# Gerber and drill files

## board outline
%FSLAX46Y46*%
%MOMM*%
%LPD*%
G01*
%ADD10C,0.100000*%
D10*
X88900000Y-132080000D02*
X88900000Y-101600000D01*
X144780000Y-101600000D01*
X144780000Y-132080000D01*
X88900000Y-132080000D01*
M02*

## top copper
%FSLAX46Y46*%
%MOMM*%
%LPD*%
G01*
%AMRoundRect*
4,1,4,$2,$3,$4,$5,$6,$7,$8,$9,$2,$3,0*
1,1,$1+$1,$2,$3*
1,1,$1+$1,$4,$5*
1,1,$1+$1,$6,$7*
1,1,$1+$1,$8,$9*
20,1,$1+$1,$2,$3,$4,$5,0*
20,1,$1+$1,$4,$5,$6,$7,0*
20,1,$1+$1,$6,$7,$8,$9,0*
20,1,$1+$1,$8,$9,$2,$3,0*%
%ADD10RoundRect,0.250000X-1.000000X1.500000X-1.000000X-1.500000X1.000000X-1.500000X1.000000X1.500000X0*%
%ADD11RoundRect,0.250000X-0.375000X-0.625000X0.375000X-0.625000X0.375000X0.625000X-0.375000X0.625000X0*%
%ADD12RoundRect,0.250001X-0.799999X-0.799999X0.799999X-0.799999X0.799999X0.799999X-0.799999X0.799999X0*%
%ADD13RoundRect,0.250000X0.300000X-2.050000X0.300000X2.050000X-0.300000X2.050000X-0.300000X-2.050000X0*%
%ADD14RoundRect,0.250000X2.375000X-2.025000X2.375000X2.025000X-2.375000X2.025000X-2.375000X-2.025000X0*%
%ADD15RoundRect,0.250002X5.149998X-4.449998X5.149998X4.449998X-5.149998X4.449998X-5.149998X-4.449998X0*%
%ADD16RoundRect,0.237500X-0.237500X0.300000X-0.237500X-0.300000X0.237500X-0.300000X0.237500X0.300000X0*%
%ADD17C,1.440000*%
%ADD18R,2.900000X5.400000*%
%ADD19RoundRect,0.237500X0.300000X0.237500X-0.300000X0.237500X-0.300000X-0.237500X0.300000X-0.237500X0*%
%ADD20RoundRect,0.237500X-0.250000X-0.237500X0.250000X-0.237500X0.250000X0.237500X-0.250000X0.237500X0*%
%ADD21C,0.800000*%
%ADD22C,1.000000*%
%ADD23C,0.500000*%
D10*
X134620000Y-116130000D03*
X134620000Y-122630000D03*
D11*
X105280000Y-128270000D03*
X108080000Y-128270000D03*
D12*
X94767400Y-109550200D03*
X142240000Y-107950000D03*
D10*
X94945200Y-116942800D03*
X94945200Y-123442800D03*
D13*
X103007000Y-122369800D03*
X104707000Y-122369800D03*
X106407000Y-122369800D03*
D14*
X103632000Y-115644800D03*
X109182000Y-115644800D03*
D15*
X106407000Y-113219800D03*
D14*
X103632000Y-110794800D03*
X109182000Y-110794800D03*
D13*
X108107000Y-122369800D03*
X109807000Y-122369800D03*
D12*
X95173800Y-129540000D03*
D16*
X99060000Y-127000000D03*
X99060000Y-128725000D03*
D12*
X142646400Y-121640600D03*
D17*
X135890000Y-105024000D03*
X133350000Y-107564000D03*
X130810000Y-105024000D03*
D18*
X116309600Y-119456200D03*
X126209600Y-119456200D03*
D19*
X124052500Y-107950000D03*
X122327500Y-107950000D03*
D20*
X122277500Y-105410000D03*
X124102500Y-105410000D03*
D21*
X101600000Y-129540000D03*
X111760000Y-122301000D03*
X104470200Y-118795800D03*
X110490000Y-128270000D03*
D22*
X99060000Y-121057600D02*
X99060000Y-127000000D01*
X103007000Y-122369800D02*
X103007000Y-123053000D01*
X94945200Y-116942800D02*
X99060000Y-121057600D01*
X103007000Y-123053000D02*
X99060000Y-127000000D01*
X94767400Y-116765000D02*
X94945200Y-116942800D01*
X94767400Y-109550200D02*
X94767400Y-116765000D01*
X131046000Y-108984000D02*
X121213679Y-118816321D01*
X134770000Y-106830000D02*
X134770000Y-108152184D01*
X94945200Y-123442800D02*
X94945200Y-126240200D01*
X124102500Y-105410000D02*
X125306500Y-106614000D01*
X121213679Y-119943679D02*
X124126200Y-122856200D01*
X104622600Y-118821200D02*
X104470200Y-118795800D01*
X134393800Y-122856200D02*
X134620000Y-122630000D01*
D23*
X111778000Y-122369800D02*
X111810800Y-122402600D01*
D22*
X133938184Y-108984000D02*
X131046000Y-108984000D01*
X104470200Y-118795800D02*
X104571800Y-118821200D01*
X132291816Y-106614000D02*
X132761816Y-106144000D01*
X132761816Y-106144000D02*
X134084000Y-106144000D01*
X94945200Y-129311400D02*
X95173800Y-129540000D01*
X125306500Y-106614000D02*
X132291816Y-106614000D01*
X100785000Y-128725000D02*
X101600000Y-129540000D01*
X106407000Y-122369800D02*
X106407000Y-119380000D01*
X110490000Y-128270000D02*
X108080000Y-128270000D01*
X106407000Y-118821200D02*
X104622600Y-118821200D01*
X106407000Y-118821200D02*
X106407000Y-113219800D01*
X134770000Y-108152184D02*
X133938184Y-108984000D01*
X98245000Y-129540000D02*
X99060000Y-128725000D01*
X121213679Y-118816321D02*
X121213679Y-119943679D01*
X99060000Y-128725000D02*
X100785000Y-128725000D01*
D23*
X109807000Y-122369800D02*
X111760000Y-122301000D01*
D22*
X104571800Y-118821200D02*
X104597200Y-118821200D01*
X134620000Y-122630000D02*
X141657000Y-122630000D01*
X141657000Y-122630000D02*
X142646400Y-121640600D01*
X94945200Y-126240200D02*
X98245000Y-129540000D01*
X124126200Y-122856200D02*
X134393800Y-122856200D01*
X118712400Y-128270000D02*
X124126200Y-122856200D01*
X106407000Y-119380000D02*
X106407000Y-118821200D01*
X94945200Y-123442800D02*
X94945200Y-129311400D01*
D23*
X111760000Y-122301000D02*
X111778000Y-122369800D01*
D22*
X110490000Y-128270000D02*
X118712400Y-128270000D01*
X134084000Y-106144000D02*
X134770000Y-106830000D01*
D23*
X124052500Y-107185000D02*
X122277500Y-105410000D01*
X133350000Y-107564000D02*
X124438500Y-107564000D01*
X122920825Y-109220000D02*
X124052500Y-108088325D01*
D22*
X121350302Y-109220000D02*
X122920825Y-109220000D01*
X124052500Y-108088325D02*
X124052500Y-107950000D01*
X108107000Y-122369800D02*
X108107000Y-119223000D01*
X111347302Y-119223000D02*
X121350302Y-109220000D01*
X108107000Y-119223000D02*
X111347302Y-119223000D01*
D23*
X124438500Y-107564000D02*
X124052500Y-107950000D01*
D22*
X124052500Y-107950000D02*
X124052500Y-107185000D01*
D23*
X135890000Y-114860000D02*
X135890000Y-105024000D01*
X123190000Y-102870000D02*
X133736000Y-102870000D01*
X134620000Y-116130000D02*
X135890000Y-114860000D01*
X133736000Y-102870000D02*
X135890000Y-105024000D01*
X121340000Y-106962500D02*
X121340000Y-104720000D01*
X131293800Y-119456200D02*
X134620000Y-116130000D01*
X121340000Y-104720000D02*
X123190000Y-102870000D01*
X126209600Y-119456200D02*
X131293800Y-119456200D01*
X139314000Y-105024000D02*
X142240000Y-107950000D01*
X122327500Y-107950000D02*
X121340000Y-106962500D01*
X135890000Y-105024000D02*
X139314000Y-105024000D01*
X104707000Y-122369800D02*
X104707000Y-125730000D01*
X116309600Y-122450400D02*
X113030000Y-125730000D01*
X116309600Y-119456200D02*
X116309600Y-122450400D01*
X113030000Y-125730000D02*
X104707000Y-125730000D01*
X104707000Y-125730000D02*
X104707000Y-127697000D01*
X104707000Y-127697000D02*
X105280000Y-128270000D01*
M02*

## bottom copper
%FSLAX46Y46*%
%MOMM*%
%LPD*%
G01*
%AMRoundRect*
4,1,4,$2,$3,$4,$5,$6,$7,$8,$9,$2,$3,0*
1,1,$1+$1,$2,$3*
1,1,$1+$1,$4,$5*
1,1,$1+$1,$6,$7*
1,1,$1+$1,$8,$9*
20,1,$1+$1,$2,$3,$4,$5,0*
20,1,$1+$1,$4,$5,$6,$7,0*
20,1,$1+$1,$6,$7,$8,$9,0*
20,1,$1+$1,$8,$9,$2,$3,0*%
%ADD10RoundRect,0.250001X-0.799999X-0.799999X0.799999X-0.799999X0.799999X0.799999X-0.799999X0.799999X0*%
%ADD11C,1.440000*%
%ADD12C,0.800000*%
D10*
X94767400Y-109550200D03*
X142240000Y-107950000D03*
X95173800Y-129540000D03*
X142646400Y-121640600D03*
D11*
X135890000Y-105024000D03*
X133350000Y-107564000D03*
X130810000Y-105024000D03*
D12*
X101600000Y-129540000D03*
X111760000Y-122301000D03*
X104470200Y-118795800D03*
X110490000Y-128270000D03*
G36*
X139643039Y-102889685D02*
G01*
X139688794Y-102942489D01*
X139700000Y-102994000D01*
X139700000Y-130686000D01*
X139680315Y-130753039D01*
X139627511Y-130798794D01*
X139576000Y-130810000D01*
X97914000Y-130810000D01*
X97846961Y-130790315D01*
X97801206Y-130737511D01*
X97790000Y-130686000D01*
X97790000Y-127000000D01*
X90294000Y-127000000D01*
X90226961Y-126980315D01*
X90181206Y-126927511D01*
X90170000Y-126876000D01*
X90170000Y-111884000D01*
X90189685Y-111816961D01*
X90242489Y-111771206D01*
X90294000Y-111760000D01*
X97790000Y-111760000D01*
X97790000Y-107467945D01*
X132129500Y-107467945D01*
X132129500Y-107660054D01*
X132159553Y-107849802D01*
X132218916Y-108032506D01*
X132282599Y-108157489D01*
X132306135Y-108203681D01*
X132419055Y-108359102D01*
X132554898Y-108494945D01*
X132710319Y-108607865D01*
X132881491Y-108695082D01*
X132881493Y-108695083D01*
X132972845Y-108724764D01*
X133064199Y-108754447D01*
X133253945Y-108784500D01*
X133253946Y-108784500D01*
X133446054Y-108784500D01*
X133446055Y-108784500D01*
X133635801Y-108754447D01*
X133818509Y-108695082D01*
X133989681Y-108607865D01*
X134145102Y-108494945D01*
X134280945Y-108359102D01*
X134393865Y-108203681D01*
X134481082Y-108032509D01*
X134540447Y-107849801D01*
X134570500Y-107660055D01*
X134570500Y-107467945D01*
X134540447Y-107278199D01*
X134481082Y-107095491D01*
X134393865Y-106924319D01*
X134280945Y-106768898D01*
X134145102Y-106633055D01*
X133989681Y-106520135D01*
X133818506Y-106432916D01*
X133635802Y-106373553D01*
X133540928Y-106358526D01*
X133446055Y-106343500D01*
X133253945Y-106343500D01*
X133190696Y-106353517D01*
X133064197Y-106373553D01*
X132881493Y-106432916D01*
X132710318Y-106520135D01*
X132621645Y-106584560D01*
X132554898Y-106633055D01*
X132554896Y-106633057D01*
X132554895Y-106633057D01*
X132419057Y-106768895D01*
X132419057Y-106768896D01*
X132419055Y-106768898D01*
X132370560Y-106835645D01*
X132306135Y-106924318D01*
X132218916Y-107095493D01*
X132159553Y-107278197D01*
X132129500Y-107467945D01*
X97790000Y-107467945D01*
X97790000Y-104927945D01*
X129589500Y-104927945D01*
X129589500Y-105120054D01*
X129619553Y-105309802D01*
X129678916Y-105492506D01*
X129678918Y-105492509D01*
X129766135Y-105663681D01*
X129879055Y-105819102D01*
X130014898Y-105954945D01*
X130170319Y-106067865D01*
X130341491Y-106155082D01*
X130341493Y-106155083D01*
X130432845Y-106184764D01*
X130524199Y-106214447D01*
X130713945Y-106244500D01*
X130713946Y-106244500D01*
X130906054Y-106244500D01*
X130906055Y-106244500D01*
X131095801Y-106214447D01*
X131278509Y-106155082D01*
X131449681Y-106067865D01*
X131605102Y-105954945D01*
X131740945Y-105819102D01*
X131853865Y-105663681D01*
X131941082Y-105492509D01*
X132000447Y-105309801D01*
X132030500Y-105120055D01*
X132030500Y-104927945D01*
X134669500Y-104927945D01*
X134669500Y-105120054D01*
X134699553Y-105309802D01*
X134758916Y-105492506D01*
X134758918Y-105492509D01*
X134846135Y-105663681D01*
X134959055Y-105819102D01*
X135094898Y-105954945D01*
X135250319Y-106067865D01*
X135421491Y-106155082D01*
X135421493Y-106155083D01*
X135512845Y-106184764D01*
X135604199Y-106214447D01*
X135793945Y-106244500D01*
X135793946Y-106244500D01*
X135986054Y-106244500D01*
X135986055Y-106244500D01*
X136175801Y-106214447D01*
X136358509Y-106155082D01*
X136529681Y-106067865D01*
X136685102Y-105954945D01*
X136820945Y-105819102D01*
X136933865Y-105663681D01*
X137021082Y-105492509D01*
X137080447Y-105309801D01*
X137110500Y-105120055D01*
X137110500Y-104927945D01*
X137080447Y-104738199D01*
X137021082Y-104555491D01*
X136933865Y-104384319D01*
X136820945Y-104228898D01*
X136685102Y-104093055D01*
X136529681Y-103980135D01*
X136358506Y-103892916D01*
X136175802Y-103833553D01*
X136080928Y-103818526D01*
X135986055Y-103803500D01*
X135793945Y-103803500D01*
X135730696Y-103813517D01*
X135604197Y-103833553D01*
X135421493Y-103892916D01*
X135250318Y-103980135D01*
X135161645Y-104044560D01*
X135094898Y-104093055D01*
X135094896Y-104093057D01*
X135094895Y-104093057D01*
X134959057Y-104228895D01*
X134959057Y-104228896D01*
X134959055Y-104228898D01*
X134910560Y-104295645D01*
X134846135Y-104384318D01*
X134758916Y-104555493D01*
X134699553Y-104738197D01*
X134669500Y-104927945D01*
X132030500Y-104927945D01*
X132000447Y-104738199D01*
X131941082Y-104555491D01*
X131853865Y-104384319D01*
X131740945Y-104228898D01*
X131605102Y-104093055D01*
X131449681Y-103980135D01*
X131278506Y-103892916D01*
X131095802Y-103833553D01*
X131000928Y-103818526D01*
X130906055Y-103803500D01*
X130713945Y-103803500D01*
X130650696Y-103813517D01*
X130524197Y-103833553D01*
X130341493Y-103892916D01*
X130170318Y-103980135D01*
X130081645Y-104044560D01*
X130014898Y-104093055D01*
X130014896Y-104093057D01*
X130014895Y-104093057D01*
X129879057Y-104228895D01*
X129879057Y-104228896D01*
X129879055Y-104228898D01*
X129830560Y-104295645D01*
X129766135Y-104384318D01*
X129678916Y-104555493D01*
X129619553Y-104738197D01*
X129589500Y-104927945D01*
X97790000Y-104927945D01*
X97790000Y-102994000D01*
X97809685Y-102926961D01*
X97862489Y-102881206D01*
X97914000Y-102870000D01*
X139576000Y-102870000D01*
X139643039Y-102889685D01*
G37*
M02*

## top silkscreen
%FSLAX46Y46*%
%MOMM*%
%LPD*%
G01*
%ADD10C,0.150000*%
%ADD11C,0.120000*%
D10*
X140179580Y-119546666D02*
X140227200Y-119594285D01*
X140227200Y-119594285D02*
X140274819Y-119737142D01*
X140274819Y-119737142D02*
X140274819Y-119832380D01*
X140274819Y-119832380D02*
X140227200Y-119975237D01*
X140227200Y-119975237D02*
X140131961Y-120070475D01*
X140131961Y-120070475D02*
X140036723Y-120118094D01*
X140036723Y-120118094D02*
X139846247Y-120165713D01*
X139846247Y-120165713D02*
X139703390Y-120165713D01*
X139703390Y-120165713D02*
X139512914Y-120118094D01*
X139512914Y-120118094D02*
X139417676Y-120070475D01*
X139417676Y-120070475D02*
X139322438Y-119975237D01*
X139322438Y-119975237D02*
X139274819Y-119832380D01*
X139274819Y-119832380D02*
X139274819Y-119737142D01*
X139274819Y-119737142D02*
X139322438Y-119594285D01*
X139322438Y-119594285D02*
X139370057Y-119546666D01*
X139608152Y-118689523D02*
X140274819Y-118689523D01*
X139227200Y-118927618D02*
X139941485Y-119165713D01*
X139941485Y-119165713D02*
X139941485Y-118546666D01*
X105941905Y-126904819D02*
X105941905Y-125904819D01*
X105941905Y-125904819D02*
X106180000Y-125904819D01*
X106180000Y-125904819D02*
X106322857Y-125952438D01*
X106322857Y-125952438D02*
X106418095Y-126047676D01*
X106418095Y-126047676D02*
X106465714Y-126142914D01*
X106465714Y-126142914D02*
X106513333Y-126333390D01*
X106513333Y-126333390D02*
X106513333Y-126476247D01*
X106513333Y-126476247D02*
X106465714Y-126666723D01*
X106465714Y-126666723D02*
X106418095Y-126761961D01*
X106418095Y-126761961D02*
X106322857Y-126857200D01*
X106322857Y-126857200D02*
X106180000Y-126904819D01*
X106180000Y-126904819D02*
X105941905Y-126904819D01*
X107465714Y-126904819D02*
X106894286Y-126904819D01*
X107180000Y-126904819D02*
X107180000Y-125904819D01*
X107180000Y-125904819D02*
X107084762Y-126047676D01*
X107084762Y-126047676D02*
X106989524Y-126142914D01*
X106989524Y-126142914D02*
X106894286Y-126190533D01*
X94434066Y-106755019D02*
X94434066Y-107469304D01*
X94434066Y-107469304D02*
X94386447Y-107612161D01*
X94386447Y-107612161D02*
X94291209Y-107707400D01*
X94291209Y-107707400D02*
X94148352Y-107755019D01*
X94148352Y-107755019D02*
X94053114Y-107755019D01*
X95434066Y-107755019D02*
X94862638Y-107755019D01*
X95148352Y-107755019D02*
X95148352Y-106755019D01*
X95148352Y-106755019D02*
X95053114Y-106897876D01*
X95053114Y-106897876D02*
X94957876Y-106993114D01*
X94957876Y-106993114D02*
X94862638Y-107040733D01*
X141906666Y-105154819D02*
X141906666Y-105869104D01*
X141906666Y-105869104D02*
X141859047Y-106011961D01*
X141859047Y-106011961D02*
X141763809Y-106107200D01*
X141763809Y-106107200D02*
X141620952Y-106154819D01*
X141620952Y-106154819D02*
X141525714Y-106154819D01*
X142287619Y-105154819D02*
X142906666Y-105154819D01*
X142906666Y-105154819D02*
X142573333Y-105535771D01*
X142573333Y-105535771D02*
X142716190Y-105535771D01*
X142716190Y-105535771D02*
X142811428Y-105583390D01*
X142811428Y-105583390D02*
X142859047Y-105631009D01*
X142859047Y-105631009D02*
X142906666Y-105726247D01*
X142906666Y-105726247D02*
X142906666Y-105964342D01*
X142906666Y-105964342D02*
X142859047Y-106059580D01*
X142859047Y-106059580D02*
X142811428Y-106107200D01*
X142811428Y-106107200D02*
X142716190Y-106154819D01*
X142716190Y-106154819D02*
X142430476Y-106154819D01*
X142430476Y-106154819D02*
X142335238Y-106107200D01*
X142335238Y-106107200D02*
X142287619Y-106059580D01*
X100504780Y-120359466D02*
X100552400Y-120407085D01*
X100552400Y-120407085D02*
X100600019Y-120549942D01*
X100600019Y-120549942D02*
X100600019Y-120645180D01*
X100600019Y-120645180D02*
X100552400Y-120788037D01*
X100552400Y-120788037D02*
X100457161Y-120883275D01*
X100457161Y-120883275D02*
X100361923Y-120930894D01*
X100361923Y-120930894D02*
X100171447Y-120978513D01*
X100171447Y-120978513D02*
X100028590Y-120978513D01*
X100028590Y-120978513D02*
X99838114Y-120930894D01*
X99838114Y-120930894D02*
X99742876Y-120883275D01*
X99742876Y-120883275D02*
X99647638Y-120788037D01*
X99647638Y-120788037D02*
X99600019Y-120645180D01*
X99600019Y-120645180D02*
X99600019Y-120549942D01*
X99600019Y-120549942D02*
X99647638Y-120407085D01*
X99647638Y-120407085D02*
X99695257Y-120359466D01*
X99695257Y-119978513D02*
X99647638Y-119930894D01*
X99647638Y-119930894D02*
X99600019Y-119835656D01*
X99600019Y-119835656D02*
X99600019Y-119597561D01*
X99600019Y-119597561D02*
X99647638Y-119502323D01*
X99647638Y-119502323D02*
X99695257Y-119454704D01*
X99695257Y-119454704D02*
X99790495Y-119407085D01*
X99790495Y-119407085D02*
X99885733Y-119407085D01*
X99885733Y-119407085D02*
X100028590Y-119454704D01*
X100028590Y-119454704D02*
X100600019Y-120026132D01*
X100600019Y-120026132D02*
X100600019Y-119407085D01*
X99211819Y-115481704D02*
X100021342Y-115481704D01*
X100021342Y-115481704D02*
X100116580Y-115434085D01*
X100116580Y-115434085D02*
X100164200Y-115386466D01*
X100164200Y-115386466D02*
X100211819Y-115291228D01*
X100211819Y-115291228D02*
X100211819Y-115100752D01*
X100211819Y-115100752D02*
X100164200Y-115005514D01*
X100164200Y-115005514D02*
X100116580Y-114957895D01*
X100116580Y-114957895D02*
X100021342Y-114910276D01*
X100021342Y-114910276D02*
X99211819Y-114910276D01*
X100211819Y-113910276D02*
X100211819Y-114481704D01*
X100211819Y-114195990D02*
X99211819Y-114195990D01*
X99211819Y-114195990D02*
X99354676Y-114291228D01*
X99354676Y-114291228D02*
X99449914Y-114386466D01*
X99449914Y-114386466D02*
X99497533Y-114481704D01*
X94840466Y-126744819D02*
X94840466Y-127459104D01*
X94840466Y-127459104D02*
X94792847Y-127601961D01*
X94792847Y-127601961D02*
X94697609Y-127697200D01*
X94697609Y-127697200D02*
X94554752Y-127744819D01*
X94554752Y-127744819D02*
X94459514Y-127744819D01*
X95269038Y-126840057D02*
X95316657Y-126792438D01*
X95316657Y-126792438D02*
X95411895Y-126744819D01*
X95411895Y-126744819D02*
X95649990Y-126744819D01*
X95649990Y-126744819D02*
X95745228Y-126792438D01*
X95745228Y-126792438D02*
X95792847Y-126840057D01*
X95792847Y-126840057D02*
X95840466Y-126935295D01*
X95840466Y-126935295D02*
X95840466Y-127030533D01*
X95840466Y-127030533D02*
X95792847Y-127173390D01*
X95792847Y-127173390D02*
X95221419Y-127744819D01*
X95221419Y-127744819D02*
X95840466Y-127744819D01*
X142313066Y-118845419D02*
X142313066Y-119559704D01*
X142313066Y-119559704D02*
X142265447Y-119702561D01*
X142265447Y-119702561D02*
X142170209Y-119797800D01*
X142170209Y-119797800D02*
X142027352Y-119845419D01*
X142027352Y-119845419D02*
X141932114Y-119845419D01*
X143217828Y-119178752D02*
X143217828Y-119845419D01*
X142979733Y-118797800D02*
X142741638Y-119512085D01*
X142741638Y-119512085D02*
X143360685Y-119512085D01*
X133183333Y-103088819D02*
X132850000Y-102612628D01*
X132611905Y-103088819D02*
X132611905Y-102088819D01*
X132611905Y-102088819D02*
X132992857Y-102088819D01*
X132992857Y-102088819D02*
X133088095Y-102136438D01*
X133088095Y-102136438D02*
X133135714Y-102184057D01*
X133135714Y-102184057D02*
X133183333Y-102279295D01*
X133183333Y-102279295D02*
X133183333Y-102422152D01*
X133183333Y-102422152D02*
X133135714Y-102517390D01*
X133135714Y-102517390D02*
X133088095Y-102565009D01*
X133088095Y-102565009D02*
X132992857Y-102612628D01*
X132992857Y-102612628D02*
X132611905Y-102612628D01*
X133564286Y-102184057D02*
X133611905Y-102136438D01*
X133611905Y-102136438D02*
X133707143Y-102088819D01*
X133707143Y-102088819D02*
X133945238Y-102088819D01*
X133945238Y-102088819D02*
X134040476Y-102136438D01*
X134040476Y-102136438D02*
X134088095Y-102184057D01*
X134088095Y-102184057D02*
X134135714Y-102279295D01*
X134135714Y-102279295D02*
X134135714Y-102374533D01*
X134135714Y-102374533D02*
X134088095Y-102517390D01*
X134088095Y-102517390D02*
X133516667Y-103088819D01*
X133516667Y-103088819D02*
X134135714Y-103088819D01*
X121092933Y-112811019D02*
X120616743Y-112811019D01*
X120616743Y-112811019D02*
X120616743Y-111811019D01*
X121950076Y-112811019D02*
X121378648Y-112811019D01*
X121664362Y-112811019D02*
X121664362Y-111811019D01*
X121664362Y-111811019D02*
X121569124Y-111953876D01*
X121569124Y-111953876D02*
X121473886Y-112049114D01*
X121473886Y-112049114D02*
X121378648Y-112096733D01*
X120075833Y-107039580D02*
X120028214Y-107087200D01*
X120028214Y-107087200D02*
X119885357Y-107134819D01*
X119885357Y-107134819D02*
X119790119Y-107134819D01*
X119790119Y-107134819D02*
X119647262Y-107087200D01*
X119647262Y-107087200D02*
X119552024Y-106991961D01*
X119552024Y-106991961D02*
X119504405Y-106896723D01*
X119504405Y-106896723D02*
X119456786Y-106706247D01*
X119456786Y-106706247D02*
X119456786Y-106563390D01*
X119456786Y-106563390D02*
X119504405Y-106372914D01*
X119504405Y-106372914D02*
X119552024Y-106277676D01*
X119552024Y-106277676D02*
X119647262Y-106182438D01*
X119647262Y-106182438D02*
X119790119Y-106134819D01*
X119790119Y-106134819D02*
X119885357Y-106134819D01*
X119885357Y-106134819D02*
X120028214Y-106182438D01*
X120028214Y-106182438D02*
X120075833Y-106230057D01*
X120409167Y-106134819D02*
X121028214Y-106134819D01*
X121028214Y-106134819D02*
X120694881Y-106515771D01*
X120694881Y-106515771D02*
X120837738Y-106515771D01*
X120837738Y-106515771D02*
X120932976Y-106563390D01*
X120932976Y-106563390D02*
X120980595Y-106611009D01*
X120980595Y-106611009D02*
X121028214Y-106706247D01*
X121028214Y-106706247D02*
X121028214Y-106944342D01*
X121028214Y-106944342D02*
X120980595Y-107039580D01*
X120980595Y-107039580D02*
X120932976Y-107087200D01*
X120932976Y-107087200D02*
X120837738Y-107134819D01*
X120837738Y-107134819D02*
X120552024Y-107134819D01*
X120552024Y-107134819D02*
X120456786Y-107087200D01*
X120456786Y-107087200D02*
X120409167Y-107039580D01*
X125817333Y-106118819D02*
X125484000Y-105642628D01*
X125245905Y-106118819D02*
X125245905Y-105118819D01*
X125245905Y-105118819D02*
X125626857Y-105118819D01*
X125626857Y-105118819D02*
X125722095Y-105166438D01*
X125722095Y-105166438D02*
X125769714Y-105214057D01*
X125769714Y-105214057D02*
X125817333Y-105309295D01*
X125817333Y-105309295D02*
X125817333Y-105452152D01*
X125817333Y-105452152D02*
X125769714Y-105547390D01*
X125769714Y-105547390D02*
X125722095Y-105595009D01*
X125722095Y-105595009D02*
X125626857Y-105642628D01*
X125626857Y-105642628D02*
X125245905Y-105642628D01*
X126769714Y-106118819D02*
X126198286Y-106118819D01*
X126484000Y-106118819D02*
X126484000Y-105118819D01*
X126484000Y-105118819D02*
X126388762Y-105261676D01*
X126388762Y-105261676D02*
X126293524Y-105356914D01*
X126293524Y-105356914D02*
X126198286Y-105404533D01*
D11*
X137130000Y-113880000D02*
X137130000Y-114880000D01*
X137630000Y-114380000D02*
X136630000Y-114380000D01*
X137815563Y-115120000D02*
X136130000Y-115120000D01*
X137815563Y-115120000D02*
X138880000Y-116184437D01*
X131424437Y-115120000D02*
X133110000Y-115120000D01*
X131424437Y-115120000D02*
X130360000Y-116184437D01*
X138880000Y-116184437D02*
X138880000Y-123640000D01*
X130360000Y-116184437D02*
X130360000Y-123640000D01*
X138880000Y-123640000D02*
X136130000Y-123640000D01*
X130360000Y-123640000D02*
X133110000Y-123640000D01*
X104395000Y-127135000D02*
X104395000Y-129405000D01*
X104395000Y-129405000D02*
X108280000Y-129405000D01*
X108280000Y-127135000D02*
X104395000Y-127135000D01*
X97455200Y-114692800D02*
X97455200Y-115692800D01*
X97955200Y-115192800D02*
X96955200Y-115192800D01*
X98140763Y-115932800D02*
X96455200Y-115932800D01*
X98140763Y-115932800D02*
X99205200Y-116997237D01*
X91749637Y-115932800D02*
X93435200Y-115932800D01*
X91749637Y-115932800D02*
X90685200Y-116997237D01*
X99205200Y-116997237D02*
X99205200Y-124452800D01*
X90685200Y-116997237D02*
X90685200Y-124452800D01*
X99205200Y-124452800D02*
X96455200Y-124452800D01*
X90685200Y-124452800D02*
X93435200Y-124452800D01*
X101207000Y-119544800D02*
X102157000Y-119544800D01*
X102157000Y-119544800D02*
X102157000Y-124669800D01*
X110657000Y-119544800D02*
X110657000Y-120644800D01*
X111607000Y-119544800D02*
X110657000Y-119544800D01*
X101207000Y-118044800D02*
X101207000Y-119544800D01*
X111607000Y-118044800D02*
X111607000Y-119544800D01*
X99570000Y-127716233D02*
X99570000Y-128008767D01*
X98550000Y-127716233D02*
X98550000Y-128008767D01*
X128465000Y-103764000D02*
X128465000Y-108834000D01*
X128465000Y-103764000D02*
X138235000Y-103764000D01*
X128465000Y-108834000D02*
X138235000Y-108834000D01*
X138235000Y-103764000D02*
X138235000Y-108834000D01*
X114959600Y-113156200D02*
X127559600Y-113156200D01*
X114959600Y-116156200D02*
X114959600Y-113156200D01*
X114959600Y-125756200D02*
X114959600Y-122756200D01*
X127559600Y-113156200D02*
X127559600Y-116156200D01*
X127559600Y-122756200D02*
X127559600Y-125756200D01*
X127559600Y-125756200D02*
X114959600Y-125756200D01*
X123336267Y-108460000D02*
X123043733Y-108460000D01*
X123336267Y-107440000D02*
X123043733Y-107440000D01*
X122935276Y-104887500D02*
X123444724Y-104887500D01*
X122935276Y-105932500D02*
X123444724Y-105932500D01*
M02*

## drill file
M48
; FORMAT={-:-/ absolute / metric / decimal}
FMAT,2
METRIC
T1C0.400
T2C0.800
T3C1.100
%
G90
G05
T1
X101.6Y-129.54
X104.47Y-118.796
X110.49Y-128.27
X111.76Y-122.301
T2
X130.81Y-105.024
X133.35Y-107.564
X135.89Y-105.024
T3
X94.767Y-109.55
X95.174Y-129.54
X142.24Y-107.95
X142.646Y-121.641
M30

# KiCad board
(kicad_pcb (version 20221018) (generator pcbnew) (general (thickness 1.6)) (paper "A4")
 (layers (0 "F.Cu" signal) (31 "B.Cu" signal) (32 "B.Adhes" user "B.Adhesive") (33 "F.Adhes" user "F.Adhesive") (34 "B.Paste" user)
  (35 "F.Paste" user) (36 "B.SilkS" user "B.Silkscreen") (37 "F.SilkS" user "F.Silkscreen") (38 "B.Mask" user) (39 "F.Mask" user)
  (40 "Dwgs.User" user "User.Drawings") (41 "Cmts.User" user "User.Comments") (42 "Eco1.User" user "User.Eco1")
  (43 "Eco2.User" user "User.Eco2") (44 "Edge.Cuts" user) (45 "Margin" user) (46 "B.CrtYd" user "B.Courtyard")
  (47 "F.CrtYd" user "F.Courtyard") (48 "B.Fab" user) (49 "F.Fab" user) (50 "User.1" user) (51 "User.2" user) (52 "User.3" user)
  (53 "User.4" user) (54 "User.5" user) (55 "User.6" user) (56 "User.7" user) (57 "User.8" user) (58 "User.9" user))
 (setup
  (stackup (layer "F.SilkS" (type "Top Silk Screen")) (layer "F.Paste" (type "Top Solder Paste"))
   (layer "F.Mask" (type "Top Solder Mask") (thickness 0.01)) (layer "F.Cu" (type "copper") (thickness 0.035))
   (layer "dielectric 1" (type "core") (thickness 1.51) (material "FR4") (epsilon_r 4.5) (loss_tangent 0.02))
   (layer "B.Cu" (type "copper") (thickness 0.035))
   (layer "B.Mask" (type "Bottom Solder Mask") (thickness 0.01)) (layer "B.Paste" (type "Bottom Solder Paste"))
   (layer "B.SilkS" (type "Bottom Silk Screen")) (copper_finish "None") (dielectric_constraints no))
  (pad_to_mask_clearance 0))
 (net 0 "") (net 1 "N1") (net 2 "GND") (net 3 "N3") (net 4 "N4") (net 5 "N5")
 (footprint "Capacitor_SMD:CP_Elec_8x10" (layer "F.Cu") (at 134.62 119.38 -90)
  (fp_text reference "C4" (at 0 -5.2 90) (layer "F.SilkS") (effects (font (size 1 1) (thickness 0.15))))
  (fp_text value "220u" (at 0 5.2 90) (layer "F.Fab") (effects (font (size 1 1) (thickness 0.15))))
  (fp_line (start -5.5 -2.51) (end -4.5 -2.51) (stroke (width 0.12) (type solid)) (layer "F.SilkS"))
  (fp_line (start -5 -3.01) (end -5 -2.01) (stroke (width 0.12) (type solid)) (layer "F.SilkS"))
  (fp_line (start -4.26 -3.195563) (end -4.26 -1.51) (stroke (width 0.12) (type solid)) (layer "F.SilkS"))
  (fp_line (start -4.26 -3.195563) (end -3.195563 -4.26) (stroke (width 0.12) (type solid)) (layer "F.SilkS"))
  (fp_line (start -4.26 3.195563) (end -4.26 1.51) (stroke (width 0.12) (type solid)) (layer "F.SilkS"))
  (fp_line (start -4.26 3.195563) (end -3.195563 4.26) (stroke (width 0.12) (type solid)) (layer "F.SilkS"))
  (fp_line (start -3.195563 -4.26) (end 4.26 -4.26) (stroke (width 0.12) (type solid)) (layer "F.SilkS"))
  (fp_line (start -3.195563 4.26) (end 4.26 4.26) (stroke (width 0.12) (type solid)) (layer "F.SilkS"))
  (fp_line (start 4.26 -4.26) (end 4.26 -1.51) (stroke (width 0.12) (type solid)) (layer "F.SilkS"))
  (fp_line (start 4.26 4.26) (end 4.26 1.51) (stroke (width 0.12) (type solid)) (layer "F.SilkS"))
  (pad "1" smd roundrect (at -3.25 0 270) (size 3.5 2.5) (layers "F.Cu" "F.Paste" "F.Mask") (roundrect_rratio 0.1) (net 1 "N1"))
  (pad "2" smd roundrect (at 3.25 0 270) (size 3.5 2.5) (layers "F.Cu" "F.Paste" "F.Mask") (roundrect_rratio 0.1) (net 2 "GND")))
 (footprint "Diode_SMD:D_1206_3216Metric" (layer "F.Cu") (at 106.68 128.27)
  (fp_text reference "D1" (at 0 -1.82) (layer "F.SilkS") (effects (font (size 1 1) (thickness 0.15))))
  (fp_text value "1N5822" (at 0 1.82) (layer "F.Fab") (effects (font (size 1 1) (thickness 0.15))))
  (fp_line (start -2.285 -1.135) (end -2.285 1.135) (stroke (width 0.12) (type solid)) (layer "F.SilkS"))
  (fp_line (start -2.285 1.135) (end 1.6 1.135) (stroke (width 0.12) (type solid)) (layer "F.SilkS"))
  (fp_line (start 1.6 -1.135) (end -2.285 -1.135) (stroke (width 0.12) (type solid)) (layer "F.SilkS"))
  (pad "1" smd roundrect (at -1.4 0) (size 1.25 1.75) (layers "F.Cu" "F.Paste" "F.Mask") (roundrect_rratio 0.2) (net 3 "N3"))
  (pad "2" smd roundrect (at 1.4 0) (size 1.25 1.75) (layers "F.Cu" "F.Paste" "F.Mask") (roundrect_rratio 0.2) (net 2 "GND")))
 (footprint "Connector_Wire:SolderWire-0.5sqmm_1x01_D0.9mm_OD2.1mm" (layer "F.Cu") (at 94.7674 109.5502)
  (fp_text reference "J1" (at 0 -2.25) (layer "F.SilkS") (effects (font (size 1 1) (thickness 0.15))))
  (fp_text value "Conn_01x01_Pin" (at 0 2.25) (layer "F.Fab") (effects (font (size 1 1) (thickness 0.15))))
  (pad "1" thru_hole roundrect (at 0 0) (size 2.1 2.1) (drill 1.1) (layers "*.Cu" "*.Mask") (roundrect_rratio 0.119048) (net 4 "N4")))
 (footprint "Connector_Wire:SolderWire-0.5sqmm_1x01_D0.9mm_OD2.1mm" (layer "F.Cu") (at 142.24 107.95)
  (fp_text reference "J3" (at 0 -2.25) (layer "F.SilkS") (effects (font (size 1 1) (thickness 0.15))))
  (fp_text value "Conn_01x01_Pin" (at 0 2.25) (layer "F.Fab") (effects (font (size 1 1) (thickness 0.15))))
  (pad "1" thru_hole roundrect (at 0 0) (size 2.1 2.1) (drill 1.1) (layers "*.Cu" "*.Mask") (roundrect_rratio 0.119048) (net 1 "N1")))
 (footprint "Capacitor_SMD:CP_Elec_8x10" (layer "F.Cu") (at 94.9452 120.1928 -90)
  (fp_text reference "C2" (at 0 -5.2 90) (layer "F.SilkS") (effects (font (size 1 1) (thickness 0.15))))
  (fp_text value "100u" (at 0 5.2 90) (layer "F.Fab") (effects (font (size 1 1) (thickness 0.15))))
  (fp_line (start -5.5 -2.51) (end -4.5 -2.51) (stroke (width 0.12) (type solid)) (layer "F.SilkS"))
  (fp_line (start -5 -3.01) (end -5 -2.01) (stroke (width 0.12) (type solid)) (layer "F.SilkS"))
  (fp_line (start -4.26 -3.195563) (end -4.26 -1.51) (stroke (width 0.12) (type solid)) (layer "F.SilkS"))
  (fp_line (start -4.26 -3.195563) (end -3.195563 -4.26) (stroke (width 0.12) (type solid)) (layer "F.SilkS"))
  (fp_line (start -4.26 3.195563) (end -4.26 1.51) (stroke (width 0.12) (type solid)) (layer "F.SilkS"))
  (fp_line (start -4.26 3.195563) (end -3.195563 4.26) (stroke (width 0.12) (type solid)) (layer "F.SilkS"))
  (fp_line (start -3.195563 -4.26) (end 4.26 -4.26) (stroke (width 0.12) (type solid)) (layer "F.SilkS"))
  (fp_line (start -3.195563 4.26) (end 4.26 4.26) (stroke (width 0.12) (type solid)) (layer "F.SilkS"))
  (fp_line (start 4.26 -4.26) (end 4.26 -1.51) (stroke (width 0.12) (type solid)) (layer "F.SilkS"))
  (fp_line (start 4.26 4.26) (end 4.26 1.51) (stroke (width 0.12) (type solid)) (layer "F.SilkS"))
  (pad "1" smd roundrect (at -3.25 0 270) (size 3.5 2.5) (layers "F.Cu" "F.Paste" "F.Mask") (roundrect_rratio 0.1) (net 4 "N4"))
  (pad "2" smd roundrect (at 3.25 0 270) (size 3.5 2.5) (layers "F.Cu" "F.Paste" "F.Mask") (roundrect_rratio 0.1) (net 2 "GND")))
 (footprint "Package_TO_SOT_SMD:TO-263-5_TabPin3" (layer "F.Cu") (at 106.407 114.7198 90)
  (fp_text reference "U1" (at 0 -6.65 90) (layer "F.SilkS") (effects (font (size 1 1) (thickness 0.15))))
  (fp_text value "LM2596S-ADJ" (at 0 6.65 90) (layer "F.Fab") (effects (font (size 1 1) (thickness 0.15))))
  (fp_line (start -4.825 -5.2) (end -4.825 -4.25) (stroke (width 0.12) (type solid)) (layer "F.SilkS"))
  (fp_line (start -4.825 -4.25) (end -9.95 -4.25) (stroke (width 0.12) (type solid)) (layer "F.SilkS"))
  (fp_line (start -4.825 4.25) (end -5.925 4.25) (stroke (width 0.12) (type solid)) (layer "F.SilkS"))
  (fp_line (start -4.825 5.2) (end -4.825 4.25) (stroke (width 0.12) (type solid)) (layer "F.SilkS"))
  (fp_line (start -3.325 -5.2) (end -4.825 -5.2) (stroke (width 0.12) (type solid)) (layer "F.SilkS"))
  (fp_line (start -3.325 5.2) (end -4.825 5.2) (stroke (width 0.12) (type solid)) (layer "F.SilkS"))
  (pad "1" smd roundrect (at -7.65 -3.4 90) (size 4.6 1.1) (layers "F.Cu" "F.Paste" "F.Mask") (roundrect_rratio 0.227273) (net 4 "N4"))
  (pad "2" smd roundrect (at -7.65 -1.7 90) (size 4.6 1.1) (layers "F.Cu" "F.Paste" "F.Mask") (roundrect_rratio 0.227273) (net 3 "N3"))
  (pad "3" smd roundrect (at -7.65 0 90) (size 4.6 1.1) (layers "F.Cu" "F.Paste" "F.Mask") (roundrect_rratio 0.227273) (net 2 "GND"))
  (pad "3" smd roundrect (at -0.925 -2.775 90) (size 4.55 5.25) (layers "F.Cu" "F.Paste") (roundrect_rratio 0.054945) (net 2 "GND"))
  (pad "3" smd roundrect (at -0.925 2.775 90) (size 4.55 5.25) (layers "F.Cu" "F.Paste") (roundrect_rratio 0.054945) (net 2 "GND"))
  (pad "3" smd roundrect (at 1.5 0 90) (size 9.4 10.8) (layers "F.Cu" "F.Mask") (roundrect_rratio 0.026596) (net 2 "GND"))
  (pad "3" smd roundrect (at 3.925 -2.775 90) (size 4.55 5.25) (layers "F.Cu" "F.Paste") (roundrect_rratio 0.054945) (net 2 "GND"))
  (pad "3" smd roundrect (at 3.925 2.775 90) (size 4.55 5.25) (layers "F.Cu" "F.Paste") (roundrect_rratio 0.054945) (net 2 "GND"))
  (pad "4" smd roundrect (at -7.65 1.7 90) (size 4.6 1.1) (layers "F.Cu" "F.Paste" "F.Mask") (roundrect_rratio 0.227273) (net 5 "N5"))
  (pad "5" smd roundrect (at -7.65 3.4 90) (size 4.6 1.1) (layers "F.Cu" "F.Paste" "F.Mask") (roundrect_rratio 0.227273) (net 2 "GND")))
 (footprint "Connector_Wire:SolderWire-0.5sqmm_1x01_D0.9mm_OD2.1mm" (layer "F.Cu") (at 95.1738 129.54)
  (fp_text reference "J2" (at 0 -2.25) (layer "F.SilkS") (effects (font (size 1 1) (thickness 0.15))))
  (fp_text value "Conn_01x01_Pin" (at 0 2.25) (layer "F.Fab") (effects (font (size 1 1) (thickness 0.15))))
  (pad "1" thru_hole roundrect (at 0 0) (size 2.1 2.1) (drill 1.1) (layers "*.Cu" "*.Mask") (roundrect_rratio 0.119048) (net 2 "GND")))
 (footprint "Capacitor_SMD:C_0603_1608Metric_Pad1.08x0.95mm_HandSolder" (layer "F.Cu") (at 99.06 127.8625 -90)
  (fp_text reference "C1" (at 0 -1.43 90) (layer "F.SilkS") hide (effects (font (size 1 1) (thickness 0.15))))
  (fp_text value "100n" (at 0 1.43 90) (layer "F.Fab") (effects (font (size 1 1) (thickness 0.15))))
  (fp_line (start -0.146267 -0.51) (end 0.146267 -0.51) (stroke (width 0.12) (type solid)) (layer "F.SilkS"))
  (fp_line (start -0.146267 0.51) (end 0.146267 0.51) (stroke (width 0.12) (type solid)) (layer "F.SilkS"))
  (pad "1" smd roundrect (at -0.8625 0 270) (size 1.075 0.95) (layers "F.Cu" "F.Paste" "F.Mask") (roundrect_rratio 0.25) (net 4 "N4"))
  (pad "2" smd roundrect (at 0.8625 0 270) (size 1.075 0.95) (layers "F.Cu" "F.Paste" "F.Mask") (roundrect_rratio 0.25) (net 2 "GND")))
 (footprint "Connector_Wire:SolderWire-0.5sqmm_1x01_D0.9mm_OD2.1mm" (layer "F.Cu") (at 142.6464 121.6406)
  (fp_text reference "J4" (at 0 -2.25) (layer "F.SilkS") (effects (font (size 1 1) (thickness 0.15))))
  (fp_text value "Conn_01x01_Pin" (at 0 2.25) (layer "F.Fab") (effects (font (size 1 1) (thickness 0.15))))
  (pad "1" thru_hole roundrect (at 0 0) (size 2.1 2.1) (drill 1.1) (layers "*.Cu" "*.Mask") (roundrect_rratio 0.119048) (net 2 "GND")))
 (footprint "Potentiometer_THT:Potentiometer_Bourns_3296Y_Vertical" (layer "F.Cu") (at 135.89 105.024)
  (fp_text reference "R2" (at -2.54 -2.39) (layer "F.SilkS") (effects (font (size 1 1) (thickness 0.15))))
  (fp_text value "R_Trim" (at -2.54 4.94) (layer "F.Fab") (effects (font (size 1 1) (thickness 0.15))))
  (fp_line (start -7.425 -1.26) (end -7.425 3.81) (stroke (width 0.12) (type solid)) (layer "F.SilkS"))
  (fp_line (start -7.425 -1.26) (end 2.345 -1.26) (stroke (width 0.12) (type solid)) (layer "F.SilkS"))
  (fp_line (start -7.425 3.81) (end 2.345 3.81) (stroke (width 0.12) (type solid)) (layer "F.SilkS"))
  (fp_line (start 2.345 -1.26) (end 2.345 3.81) (stroke (width 0.12) (type solid)) (layer "F.SilkS"))
  (pad "1" thru_hole circle (at 0 0) (size 1.44 1.44) (drill 0.8) (layers "*.Cu" "*.Mask") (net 1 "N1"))
  (pad "2" thru_hole circle (at -2.54 2.54) (size 1.44 1.44) (drill 0.8) (layers "*.Cu" "*.Mask") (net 5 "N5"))
  (pad "3" thru_hole circle (at -5.08 0) (size 1.44 1.44) (drill 0.8) (layers "*.Cu" "*.Mask")))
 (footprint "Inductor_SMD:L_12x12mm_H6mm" (layer "F.Cu") (at 121.2596 119.4562)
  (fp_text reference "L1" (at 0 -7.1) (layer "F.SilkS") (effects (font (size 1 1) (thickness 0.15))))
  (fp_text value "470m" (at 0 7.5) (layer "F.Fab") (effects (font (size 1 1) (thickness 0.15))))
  (fp_line (start -6.3 -6.3) (end 6.3 -6.3) (stroke (width 0.12) (type solid)) (layer "F.SilkS"))
  (fp_line (start -6.3 -3.3) (end -6.3 -6.3) (stroke (width 0.12) (type solid)) (layer "F.SilkS"))
  (fp_line (start -6.3 6.3) (end -6.3 3.3) (stroke (width 0.12) (type solid)) (layer "F.SilkS"))
  (fp_line (start 6.3 -6.3) (end 6.3 -3.3) (stroke (width 0.12) (type solid)) (layer "F.SilkS"))
  (fp_line (start 6.3 3.3) (end 6.3 6.3) (stroke (width 0.12) (type solid)) (layer "F.SilkS"))
  (fp_line (start 6.3 6.3) (end -6.3 6.3) (stroke (width 0.12) (type solid)) (layer "F.SilkS"))
  (pad "1" smd rect (at -4.95 0) (size 2.9 5.4) (layers "F.Cu" "F.Paste" "F.Mask") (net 3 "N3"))
  (pad "2" smd rect (at 4.95 0) (size 2.9 5.4) (layers "F.Cu" "F.Paste" "F.Mask") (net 1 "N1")))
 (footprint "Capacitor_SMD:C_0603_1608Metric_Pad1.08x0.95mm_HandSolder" (layer "F.Cu") (at 123.19 107.95 180)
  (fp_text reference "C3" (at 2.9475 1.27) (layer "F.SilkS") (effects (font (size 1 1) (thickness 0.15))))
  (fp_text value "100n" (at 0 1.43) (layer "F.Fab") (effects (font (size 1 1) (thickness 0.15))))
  (fp_line (start -0.146267 -0.51) (end 0.146267 -0.51) (stroke (width 0.12) (type solid)) (layer "F.SilkS"))
  (fp_line (start -0.146267 0.51) (end 0.146267 0.51) (stroke (width 0.12) (type solid)) (layer "F.SilkS"))
  (pad "1" smd roundrect (at -0.8625 0 180) (size 1.075 0.95) (layers "F.Cu" "F.Paste" "F.Mask") (roundrect_rratio 0.25) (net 5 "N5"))
  (pad "2" smd roundrect (at 0.8625 0 180) (size 1.075 0.95) (layers "F.Cu" "F.Paste" "F.Mask") (roundrect_rratio 0.25) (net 1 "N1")))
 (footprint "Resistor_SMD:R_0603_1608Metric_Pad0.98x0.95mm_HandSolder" (layer "F.Cu") (at 123.19 105.41)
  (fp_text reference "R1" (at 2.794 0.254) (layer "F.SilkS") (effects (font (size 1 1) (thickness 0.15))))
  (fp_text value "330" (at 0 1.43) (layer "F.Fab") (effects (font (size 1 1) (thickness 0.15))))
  (fp_line (start -0.254724 -0.5225) (end 0.254724 -0.5225) (stroke (width 0.12) (type solid)) (layer "F.SilkS"))
  (fp_line (start -0.254724 0.5225) (end 0.254724 0.5225) (stroke (width 0.12) (type solid)) (layer "F.SilkS"))
  (pad "1" smd roundrect (at -0.9125 0) (size 0.975 0.95) (layers "F.Cu" "F.Paste" "F.Mask") (roundrect_rratio 0.25) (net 5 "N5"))
  (pad "2" smd roundrect (at 0.9125 0) (size 0.975 0.95) (layers "F.Cu" "F.Paste" "F.Mask") (roundrect_rratio 0.25) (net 2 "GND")))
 (gr_poly
  (pts (xy 88.9 132.08) (xy 88.9 101.6) (xy 144.78 101.6) (xy 144.78 132.08)) (stroke (width 0.1) (type solid)) (fill none)
  (layer "Edge.Cuts"))
 (segment (start 99.06 121.0576) (end 99.06 127) (width 1) (layer "F.Cu") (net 4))
 (segment (start 103.007 122.3698) (end 103.007 123.053) (width 1) (layer "F.Cu") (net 4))
 (segment (start 94.9452 116.9428) (end 99.06 121.0576) (width 1) (layer "F.Cu") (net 4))
 (segment (start 103.007 123.053) (end 99.06 127) (width 1) (layer "F.Cu") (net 4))
 (segment (start 94.7674 116.765) (end 94.9452 116.9428) (width 1) (layer "F.Cu") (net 4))
 (segment (start 94.7674 109.5502) (end 94.7674 116.765) (width 1) (layer "F.Cu") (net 4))
 (segment (start 131.046 108.984) (end 121.213679 118.816321) (width 1) (layer "F.Cu") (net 2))
 (segment (start 134.77 106.83) (end 134.77 108.152184) (width 1) (layer "F.Cu") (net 2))
 (segment (start 94.9452 123.4428) (end 94.9452 126.2402) (width 1) (layer "F.Cu") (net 2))
 (segment (start 124.1025 105.41) (end 125.3065 106.614) (width 1) (layer "F.Cu") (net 2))
 (segment (start 121.213679 119.943679) (end 124.1262 122.8562) (width 1) (layer "F.Cu") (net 2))
 (segment (start 104.6226 118.8212) (end 104.4702 118.7958) (width 1) (layer "F.Cu") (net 2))
 (segment (start 134.3938 122.8562) (end 134.62 122.63) (width 1) (layer "F.Cu") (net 2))
 (segment (start 111.778 122.3698) (end 111.8108 122.4026) (width 0.5) (layer "F.Cu") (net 2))
 (segment (start 133.938184 108.984) (end 131.046 108.984) (width 1) (layer "F.Cu") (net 2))
 (segment (start 104.4702 118.7958) (end 104.5718 118.8212) (width 1) (layer "F.Cu") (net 2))
 (segment (start 132.291816 106.614) (end 132.761816 106.144) (width 1) (layer "F.Cu") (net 2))
 (segment (start 132.761816 106.144) (end 134.084 106.144) (width 1) (layer "F.Cu") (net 2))
 (segment (start 94.9452 129.3114) (end 95.1738 129.54) (width 1) (layer "F.Cu") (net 2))
 (segment (start 125.3065 106.614) (end 132.291816 106.614) (width 1) (layer "F.Cu") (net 2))
 (segment (start 100.785 128.725) (end 101.6 129.54) (width 1) (layer "F.Cu") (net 2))
 (segment (start 106.407 122.3698) (end 106.407 119.38) (width 1) (layer "F.Cu") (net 2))
 (segment (start 110.49 128.27) (end 108.08 128.27) (width 1) (layer "F.Cu") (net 2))
 (segment (start 106.407 118.8212) (end 104.6226 118.8212) (width 1) (layer "F.Cu") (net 2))
 (segment (start 106.407 118.8212) (end 106.407 113.2198) (width 1) (layer "F.Cu") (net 2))
 (segment (start 134.77 108.152184) (end 133.938184 108.984) (width 1) (layer "F.Cu") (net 2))
 (segment (start 98.245 129.54) (end 99.06 128.725) (width 1) (layer "F.Cu") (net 2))
 (segment (start 121.213679 118.816321) (end 121.213679 119.943679) (width 1) (layer "F.Cu") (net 2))
 (segment (start 99.06 128.725) (end 100.785 128.725) (width 1) (layer "F.Cu") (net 2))
 (segment (start 109.807 122.3698) (end 111.76 122.301) (width 0.5) (layer "F.Cu") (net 2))
 (segment (start 104.5718 118.8212) (end 104.5972 118.8212) (width 1) (layer "F.Cu") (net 2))
 (segment (start 134.62 122.63) (end 141.657 122.63) (width 1) (layer "F.Cu") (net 2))
 (segment (start 141.657 122.63) (end 142.6464 121.6406) (width 1) (layer "F.Cu") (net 2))
 (segment (start 94.9452 126.2402) (end 98.245 129.54) (width 1) (layer "F.Cu") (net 2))
 (segment (start 124.1262 122.8562) (end 134.3938 122.8562) (width 1) (layer "F.Cu") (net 2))
 (segment (start 118.7124 128.27) (end 124.1262 122.8562) (width 1) (layer "F.Cu") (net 2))
 (segment (start 106.407 119.38) (end 106.407 118.8212) (width 1) (layer "F.Cu") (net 2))
 (segment (start 94.9452 123.4428) (end 94.9452 129.3114) (width 1) (layer "F.Cu") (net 2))
 (segment (start 111.76 122.301) (end 111.778 122.3698) (width 0.5) (layer "F.Cu") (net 2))
 (segment (start 110.49 128.27) (end 118.7124 128.27) (width 1) (layer "F.Cu") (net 2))
 (segment (start 134.084 106.144) (end 134.77 106.83) (width 1) (layer "F.Cu") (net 2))
 (via (at 101.6 129.54) (size 0.8) (drill 0.4) (layers "F.Cu" "B.Cu") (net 2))
 (via (at 111.76 122.301) (size 0.8) (drill 0.4) (layers "F.Cu" "B.Cu") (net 2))
 (via (at 104.4702 118.7958) (size 0.8) (drill 0.4) (layers "F.Cu" "B.Cu") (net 2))
 (via (at 110.49 128.27) (size 0.8) (drill 0.4) (layers "F.Cu" "B.Cu") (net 2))
 (segment (start 124.0525 107.185) (end 122.2775 105.41) (width 0.5) (layer "F.Cu") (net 5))
 (segment (start 133.35 107.564) (end 124.4385 107.564) (width 0.5) (layer "F.Cu") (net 5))
 (segment (start 122.920825 109.22) (end 124.0525 108.088325) (width 0.5) (layer "F.Cu") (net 5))
 (segment (start 121.350302 109.22) (end 122.920825 109.22) (width 1) (layer "F.Cu") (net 5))
 (segment (start 124.0525 108.088325) (end 124.0525 107.95) (width 1) (layer "F.Cu") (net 5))
 (segment (start 108.107 122.3698) (end 108.107 119.223) (width 1) (layer "F.Cu") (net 5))
 (segment (start 111.347302 119.223) (end 121.350302 109.22) (width 1) (layer "F.Cu") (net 5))
 (segment (start 108.107 119.223) (end 111.347302 119.223) (width 1) (layer "F.Cu") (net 5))
 (segment (start 124.4385 107.564) (end 124.0525 107.95) (width 0.5) (layer "F.Cu") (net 5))
 (segment (start 124.0525 107.95) (end 124.0525 107.185) (width 1) (layer "F.Cu") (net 5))
 (segment (start 135.89 114.86) (end 135.89 105.024) (width 0.5) (layer "F.Cu") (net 1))
 (segment (start 123.19 102.87) (end 133.736 102.87) (width 0.5) (layer "F.Cu") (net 1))
 (segment (start 134.62 116.13) (end 135.89 114.86) (width 0.5) (layer "F.Cu") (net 1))
 (segment (start 133.736 102.87) (end 135.89 105.024) (width 0.5) (layer "F.Cu") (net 1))
 (segment (start 121.34 106.9625) (end 121.34 104.72) (width 0.5) (layer "F.Cu") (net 1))
 (segment (start 131.2938 119.4562) (end 134.62 116.13) (width 0.5) (layer "F.Cu") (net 1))
 (segment (start 121.34 104.72) (end 123.19 102.87) (width 0.5) (layer "F.Cu") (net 1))
 (segment (start 126.2096 119.4562) (end 131.2938 119.4562) (width 0.5) (layer "F.Cu") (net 1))
 (segment (start 139.314 105.024) (end 142.24 107.95) (width 0.5) (layer "F.Cu") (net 1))
 (segment (start 122.3275 107.95) (end 121.34 106.9625) (width 0.5) (layer "F.Cu") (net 1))
 (segment (start 135.89 105.024) (end 139.314 105.024) (width 0.5) (layer "F.Cu") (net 1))
 (segment (start 104.707 122.3698) (end 104.707 125.73) (width 0.5) (layer "F.Cu") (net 3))
 (segment (start 116.3096 122.4504) (end 113.03 125.73) (width 0.5) (layer "F.Cu") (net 3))
 (segment (start 116.3096 119.4562) (end 116.3096 122.4504) (width 0.5) (layer "F.Cu") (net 3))
 (segment (start 113.03 125.73) (end 104.707 125.73) (width 0.5) (layer "F.Cu") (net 3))
 (segment (start 104.707 125.73) (end 104.707 127.697) (width 0.5) (layer "F.Cu") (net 3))
 (segment (start 104.707 127.697) (end 105.28 128.27) (width 0.5) (layer "F.Cu") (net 3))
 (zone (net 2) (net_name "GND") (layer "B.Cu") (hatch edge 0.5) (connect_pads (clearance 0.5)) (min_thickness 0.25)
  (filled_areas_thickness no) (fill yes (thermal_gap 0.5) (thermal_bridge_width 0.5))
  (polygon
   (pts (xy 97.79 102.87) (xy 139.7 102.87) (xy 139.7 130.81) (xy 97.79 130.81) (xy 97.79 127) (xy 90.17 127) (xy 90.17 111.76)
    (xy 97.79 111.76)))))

